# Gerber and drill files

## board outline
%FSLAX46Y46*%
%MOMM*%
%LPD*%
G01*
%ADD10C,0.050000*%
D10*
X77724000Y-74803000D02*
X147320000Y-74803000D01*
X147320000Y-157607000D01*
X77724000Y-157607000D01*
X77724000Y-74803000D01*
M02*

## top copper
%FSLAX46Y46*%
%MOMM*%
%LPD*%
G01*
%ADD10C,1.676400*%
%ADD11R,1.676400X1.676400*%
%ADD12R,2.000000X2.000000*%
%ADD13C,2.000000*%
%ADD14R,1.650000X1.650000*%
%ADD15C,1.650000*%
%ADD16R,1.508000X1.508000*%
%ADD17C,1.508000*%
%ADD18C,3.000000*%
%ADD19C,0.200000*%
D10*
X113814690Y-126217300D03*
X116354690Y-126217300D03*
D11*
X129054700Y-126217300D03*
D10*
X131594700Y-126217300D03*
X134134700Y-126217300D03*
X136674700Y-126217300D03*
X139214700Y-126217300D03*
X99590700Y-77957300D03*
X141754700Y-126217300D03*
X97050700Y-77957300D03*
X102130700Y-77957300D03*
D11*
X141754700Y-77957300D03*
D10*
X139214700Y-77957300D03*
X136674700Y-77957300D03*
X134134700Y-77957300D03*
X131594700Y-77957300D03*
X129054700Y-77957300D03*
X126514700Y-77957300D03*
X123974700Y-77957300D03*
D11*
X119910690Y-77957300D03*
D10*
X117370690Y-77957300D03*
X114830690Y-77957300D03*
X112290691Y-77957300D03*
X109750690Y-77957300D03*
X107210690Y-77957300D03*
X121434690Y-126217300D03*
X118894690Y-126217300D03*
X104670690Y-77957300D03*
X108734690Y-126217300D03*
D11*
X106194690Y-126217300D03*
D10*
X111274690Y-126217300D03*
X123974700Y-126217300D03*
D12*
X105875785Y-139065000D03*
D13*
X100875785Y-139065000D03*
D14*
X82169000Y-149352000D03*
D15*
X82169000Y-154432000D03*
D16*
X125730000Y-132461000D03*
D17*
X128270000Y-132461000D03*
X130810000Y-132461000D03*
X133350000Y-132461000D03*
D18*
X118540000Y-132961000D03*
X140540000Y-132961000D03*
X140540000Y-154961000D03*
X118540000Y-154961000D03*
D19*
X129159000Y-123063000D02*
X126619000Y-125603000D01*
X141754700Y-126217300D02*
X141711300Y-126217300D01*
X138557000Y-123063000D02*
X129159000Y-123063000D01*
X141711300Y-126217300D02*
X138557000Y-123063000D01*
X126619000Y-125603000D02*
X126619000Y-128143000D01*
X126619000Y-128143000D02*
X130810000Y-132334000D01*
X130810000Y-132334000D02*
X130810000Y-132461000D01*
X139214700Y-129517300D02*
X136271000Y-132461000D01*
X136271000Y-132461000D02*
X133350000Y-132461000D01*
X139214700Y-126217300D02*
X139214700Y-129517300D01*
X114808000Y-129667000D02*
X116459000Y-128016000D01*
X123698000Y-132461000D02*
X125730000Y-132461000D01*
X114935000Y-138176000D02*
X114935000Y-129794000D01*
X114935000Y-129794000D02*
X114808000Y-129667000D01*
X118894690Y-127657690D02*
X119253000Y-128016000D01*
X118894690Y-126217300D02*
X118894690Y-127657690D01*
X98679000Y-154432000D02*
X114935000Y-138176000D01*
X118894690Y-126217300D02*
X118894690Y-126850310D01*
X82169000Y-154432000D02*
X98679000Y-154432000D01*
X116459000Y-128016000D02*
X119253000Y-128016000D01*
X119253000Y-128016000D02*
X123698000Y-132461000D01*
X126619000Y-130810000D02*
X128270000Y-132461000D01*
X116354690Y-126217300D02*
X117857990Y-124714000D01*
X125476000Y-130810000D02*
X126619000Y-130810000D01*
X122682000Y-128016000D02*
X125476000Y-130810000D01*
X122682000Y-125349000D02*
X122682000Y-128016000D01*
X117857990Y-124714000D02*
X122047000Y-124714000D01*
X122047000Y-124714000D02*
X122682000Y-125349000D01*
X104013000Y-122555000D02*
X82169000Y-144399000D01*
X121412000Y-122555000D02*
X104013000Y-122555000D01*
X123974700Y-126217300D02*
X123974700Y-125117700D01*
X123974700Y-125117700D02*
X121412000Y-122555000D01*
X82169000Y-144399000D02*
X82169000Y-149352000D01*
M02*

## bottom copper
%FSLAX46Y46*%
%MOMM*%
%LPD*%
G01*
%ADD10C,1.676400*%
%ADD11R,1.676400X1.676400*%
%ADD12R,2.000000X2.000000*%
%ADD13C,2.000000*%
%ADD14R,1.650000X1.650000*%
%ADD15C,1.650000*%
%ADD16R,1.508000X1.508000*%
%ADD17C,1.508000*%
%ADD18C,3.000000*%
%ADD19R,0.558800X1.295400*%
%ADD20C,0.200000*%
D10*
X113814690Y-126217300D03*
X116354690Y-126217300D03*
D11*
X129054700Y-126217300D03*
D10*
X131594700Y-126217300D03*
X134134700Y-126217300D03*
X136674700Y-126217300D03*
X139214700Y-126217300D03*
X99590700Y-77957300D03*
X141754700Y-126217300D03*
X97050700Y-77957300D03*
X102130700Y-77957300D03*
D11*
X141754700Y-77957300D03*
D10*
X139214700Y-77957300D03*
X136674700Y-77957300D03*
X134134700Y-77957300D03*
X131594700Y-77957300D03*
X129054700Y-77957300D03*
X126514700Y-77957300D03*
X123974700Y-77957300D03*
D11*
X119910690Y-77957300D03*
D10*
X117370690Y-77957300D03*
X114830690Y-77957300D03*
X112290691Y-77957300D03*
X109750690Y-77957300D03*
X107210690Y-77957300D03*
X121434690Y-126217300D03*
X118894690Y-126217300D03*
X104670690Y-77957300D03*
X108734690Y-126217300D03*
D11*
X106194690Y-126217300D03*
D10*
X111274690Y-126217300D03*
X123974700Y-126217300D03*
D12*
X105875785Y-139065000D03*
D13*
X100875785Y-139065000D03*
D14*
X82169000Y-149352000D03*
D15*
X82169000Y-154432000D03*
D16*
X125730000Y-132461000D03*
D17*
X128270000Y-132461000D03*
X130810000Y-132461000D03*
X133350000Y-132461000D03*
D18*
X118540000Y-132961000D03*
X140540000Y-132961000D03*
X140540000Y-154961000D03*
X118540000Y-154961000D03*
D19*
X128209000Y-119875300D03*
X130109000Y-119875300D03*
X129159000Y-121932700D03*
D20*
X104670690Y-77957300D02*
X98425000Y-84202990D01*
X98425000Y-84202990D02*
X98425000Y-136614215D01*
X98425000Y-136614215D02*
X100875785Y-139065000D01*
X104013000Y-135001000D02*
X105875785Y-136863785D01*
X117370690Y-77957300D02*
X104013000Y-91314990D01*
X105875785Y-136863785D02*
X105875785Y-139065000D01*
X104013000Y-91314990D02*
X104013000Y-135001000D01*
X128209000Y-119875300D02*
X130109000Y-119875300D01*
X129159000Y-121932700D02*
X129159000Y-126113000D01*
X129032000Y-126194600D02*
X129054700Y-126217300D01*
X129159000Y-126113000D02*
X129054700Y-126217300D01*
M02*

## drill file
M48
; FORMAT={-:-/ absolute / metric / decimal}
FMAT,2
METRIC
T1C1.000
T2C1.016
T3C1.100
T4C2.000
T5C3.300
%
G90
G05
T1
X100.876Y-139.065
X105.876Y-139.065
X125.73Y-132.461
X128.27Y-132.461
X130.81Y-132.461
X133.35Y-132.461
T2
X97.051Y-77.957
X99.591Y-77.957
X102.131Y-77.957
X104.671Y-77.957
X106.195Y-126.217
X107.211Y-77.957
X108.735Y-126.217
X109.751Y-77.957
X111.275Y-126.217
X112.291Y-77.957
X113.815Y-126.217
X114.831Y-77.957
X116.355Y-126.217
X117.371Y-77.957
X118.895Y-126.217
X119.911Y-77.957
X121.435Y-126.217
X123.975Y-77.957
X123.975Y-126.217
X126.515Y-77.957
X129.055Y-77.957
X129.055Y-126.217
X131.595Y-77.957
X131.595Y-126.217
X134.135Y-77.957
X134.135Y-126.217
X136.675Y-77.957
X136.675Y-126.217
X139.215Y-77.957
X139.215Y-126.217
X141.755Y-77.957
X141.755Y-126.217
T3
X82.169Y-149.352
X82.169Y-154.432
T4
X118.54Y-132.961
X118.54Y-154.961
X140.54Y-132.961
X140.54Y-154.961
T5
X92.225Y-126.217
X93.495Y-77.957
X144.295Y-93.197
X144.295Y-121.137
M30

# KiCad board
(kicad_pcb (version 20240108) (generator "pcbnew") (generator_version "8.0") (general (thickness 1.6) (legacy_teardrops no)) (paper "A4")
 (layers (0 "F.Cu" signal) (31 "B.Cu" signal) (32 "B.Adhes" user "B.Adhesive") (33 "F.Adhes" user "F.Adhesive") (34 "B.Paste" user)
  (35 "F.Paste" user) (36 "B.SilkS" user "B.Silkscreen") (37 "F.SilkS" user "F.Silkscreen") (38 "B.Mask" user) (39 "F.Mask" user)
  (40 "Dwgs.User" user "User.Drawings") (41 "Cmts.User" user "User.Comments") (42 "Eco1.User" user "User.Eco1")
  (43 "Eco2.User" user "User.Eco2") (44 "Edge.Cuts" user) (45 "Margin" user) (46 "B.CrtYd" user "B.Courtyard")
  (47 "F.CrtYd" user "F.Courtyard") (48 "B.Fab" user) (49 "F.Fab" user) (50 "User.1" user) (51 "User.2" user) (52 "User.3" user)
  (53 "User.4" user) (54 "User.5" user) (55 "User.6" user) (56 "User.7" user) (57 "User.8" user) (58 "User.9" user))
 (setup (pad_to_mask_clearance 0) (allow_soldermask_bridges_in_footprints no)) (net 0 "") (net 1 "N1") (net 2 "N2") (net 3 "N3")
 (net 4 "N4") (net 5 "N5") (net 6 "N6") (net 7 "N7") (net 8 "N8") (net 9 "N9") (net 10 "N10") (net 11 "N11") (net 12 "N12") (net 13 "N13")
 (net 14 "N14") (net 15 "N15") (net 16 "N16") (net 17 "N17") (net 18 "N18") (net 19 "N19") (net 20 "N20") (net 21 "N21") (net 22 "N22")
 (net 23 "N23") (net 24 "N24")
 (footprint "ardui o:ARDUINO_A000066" (layer "F.Cu") (at 112.522 102.108)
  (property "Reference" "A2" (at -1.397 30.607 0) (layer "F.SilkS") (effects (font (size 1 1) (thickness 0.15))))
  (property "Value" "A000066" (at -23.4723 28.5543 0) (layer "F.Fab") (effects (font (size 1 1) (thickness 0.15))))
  (pad "" np_thru_hole circle (at -20.2973 24.1093) (size 3.3 3.3) (drill 3.3) (layers "*.Cu" "*.Mask"))
  (pad "" np_thru_hole circle (at -19.0273 -24.1507) (size 3.3 3.3) (drill 3.3) (layers "*.Cu" "*.Mask"))
  (pad "" np_thru_hole circle (at 31.7727 -8.91069) (size 3.3 3.3) (drill 3.3) (layers "*.Cu" "*.Mask"))
  (pad "" np_thru_hole circle (at 31.7727 19.0293) (size 3.3 3.3) (drill 3.3) (layers "*.Cu" "*.Mask"))
  (pad "3V3" thru_hole circle (at 1.29269 24.1093) (size 1.6764 1.6764) (drill 1.016) (layers "*.Cu" "*.Mask") (remove_unused_layers no)
   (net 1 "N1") (solder_mask_margin 0.102))
  (pad "5V" thru_hole circle (at 3.83269 24.1093) (size 1.6764 1.6764) (drill 1.016) (layers "*.Cu" "*.Mask") (remove_unused_layers no)
   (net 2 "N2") (solder_mask_margin 0.102))
  (pad "A0" thru_hole rect (at 16.5327 24.1093) (size 1.6764 1.6764) (drill 1.016) (layers "*.Cu" "*.Mask") (remove_unused_layers no)
   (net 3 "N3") (solder_mask_margin 0.102))
  (pad "A1" thru_hole circle (at 19.0727 24.1093) (size 1.6764 1.6764) (drill 1.016) (layers "*.Cu" "*.Mask") (remove_unused_layers no)
   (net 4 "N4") (solder_mask_margin 0.102))
  (pad "A2" thru_hole circle (at 21.6127 24.1093) (size 1.6764 1.6764) (drill 1.016) (layers "*.Cu" "*.Mask") (remove_unused_layers no)
   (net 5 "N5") (solder_mask_margin 0.102))
  (pad "A3" thru_hole circle (at 24.1527 24.1093) (size 1.6764 1.6764) (drill 1.016) (layers "*.Cu" "*.Mask") (remove_unused_layers no)
   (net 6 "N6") (solder_mask_margin 0.102))
  (pad "A4" thru_hole circle (at 26.6927 24.1093) (size 1.6764 1.6764) (drill 1.016) (layers "*.Cu" "*.Mask") (remove_unused_layers no)
   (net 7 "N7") (solder_mask_margin 0.102))
  (pad "A4_SDA" thru_hole circle (at -12.9313 -24.1507) (size 1.6764 1.6764) (drill 1.016) (layers "*.Cu" "*.Mask")
   (remove_unused_layers no) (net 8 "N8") (solder_mask_margin 0.102))
  (pad "A5" thru_hole circle (at 29.2327 24.1093) (size 1.6764 1.6764) (drill 1.016) (layers "*.Cu" "*.Mask") (remove_unused_layers no)
   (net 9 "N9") (solder_mask_margin 0.102))
  (pad "A5_SCL" thru_hole circle (at -15.4713 -24.1507) (size 1.6764 1.6764) (drill 1.016) (layers "*.Cu" "*.Mask")
   (remove_unused_layers no) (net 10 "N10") (solder_mask_margin 0.102))
  (pad "AREF" thru_hole circle (at -10.3913 -24.1507) (size 1.6764 1.6764) (drill 1.016) (layers "*.Cu" "*.Mask") (remove_unused_layers no)
   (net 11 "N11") (solder_mask_margin 0.102))
  (pad "D0" thru_hole rect (at 29.2327 -24.1507) (size 1.6764 1.6764) (drill 1.016) (layers "*.Cu" "*.Mask") (remove_unused_layers no)
   (solder_mask_margin 0.102))
  (pad "D1" thru_hole circle (at 26.6927 -24.1507) (size 1.6764 1.6764) (drill 1.016) (layers "*.Cu" "*.Mask") (remove_unused_layers no)
   (solder_mask_margin 0.102))
  (pad "D2" thru_hole circle (at 24.1527 -24.1507) (size 1.6764 1.6764) (drill 1.016) (layers "*.Cu" "*.Mask") (remove_unused_layers no)
   (solder_mask_margin 0.102))
  (pad "D3" thru_hole circle (at 21.6127 -24.1507) (size 1.6764 1.6764) (drill 1.016) (layers "*.Cu" "*.Mask") (remove_unused_layers no)
   (solder_mask_margin 0.102))
  (pad "D4" thru_hole circle (at 19.0727 -24.1507) (size 1.6764 1.6764) (drill 1.016) (layers "*.Cu" "*.Mask") (remove_unused_layers no)
   (solder_mask_margin 0.102))
  (pad "D5" thru_hole circle (at 16.5327 -24.1507) (size 1.6764 1.6764) (drill 1.016) (layers "*.Cu" "*.Mask") (remove_unused_layers no)
   (solder_mask_margin 0.102))
  (pad "D6" thru_hole circle (at 13.9927 -24.1507) (size 1.6764 1.6764) (drill 1.016) (layers "*.Cu" "*.Mask") (remove_unused_layers no)
   (solder_mask_margin 0.102))
  (pad "D7" thru_hole circle (at 11.4527 -24.1507) (size 1.6764 1.6764) (drill 1.016) (layers "*.Cu" "*.Mask") (remove_unused_layers no)
   (solder_mask_margin 0.102))
  (pad "D8" thru_hole rect (at 7.38869 -24.1507) (size 1.6764 1.6764) (drill 1.016) (layers "*.Cu" "*.Mask") (remove_unused_layers no)
   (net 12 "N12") (solder_mask_margin 0.102))
  (pad "D9" thru_hole circle (at 4.84869 -24.1507) (size 1.6764 1.6764) (drill 1.016) (layers "*.Cu" "*.Mask") (remove_unused_layers no)
   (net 12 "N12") (solder_mask_margin 0.102))
  (pad "D10" thru_hole circle (at 2.30869 -24.1507) (size 1.6764 1.6764) (drill 1.016) (layers "*.Cu" "*.Mask") (remove_unused_layers no)
   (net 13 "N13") (solder_mask_margin 0.102))
  (pad "D11" thru_hole circle (at -0.231309 -24.1507) (size 1.6764 1.6764) (drill 1.016) (layers "*.Cu" "*.Mask") (remove_unused_layers no)
   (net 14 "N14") (solder_mask_margin 0.102))
  (pad "D12" thru_hole circle (at -2.77131 -24.1507) (size 1.6764 1.6764) (drill 1.016) (layers "*.Cu" "*.Mask") (remove_unused_layers no)
   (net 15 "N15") (solder_mask_margin 0.102))
  (pad "D13" thru_hole circle (at -5.31131 -24.1507) (size 1.6764 1.6764) (drill 1.016) (layers "*.Cu" "*.Mask") (remove_unused_layers no)
   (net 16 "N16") (solder_mask_margin 0.102))
  (pad "GND_1" thru_hole circle (at 8.91269 24.1093) (size 1.6764 1.6764) (drill 1.016) (layers "*.Cu" "*.Mask") (remove_unused_layers no)
   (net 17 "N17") (solder_mask_margin 0.102))
  (pad "GND_2" thru_hole circle (at 6.37269 24.1093) (size 1.6764 1.6764) (drill 1.016) (layers "*.Cu" "*.Mask") (remove_unused_layers no)
   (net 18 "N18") (solder_mask_margin 0.102))
  (pad "GND_3" thru_hole circle (at -7.85131 -24.1507) (size 1.6764 1.6764) (drill 1.016) (layers "*.Cu" "*.Mask") (remove_unused_layers no)
   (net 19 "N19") (solder_mask_margin 0.102))
  (pad "IOREF" thru_hole circle (at -3.78731 24.1093) (size 1.6764 1.6764) (drill 1.016) (layers "*.Cu" "*.Mask") (remove_unused_layers no)
   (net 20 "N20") (solder_mask_margin 0.102))
  (pad "P1" thru_hole rect (at -6.32731 24.1093) (size 1.6764 1.6764) (drill 1.016) (layers "*.Cu" "*.Mask") (remove_unused_layers no)
   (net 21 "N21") (solder_mask_margin 0.102))
  (pad "RST" thru_hole circle (at -1.24731 24.1093) (size 1.6764 1.6764) (drill 1.016) (layers "*.Cu" "*.Mask") (remove_unused_layers no)
   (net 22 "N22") (solder_mask_margin 0.102))
  (pad "VIN" thru_hole circle (at 11.4527 24.1093) (size 1.6764 1.6764) (drill 1.016) (layers "*.Cu" "*.Mask") (remove_unused_layers no)
   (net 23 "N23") (solder_mask_margin 0.102)))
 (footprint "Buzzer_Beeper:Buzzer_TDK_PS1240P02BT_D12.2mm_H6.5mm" (layer "F.Cu") (at 105.875785 139.065 180)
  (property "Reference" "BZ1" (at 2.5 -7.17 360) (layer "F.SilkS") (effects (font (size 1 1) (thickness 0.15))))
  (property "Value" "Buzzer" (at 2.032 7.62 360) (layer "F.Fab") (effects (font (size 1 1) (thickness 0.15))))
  (pad "1" thru_hole rect (at 0 0 180) (size 2 2) (drill 1) (layers "*.Cu" "*.Mask") (remove_unused_layers no) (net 12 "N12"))
  (pad "2" thru_hole circle (at 5 0 180) (size 2 2) (drill 1) (layers "*.Cu" "*.Mask") (remove_unused_layers no) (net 19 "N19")))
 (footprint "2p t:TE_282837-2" (layer "F.Cu") (at 82.169 151.892 -90)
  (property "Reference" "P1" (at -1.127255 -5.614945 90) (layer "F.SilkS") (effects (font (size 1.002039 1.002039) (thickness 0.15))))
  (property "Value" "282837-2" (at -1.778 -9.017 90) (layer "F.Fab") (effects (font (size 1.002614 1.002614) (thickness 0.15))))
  (pad "1" thru_hole rect (at -2.54 0 270) (size 1.65 1.65) (drill 1.1) (layers "*.Cu" "*.Mask") (remove_unused_layers no) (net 23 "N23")
   (solder_mask_margin 0.102))
  (pad "2" thru_hole circle (at 2.54 0 270) (size 1.65 1.65) (drill 1.1) (layers "*.Cu" "*.Mask") (remove_unused_layers no) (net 18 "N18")
   (solder_mask_margin 0.102)))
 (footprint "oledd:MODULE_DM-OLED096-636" (layer "F.Cu") (at 129.54 143.961)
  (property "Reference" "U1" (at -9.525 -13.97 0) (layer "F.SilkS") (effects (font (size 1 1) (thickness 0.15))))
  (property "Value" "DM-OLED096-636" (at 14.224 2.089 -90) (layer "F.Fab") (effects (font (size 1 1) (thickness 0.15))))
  (pad "1" thru_hole rect (at -3.81 -11.5) (size 1.508 1.508) (drill 1) (layers "*.Cu" "*.Mask") (remove_unused_layers no) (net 18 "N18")
   (solder_mask_margin 0.102))
  (pad "2" thru_hole circle (at -1.27 -11.5) (size 1.508 1.508) (drill 1) (layers "*.Cu" "*.Mask") (remove_unused_layers no) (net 2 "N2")
   (solder_mask_margin 0.102))
  (pad "3" thru_hole circle (at 1.27 -11.5) (size 1.508 1.508) (drill 1) (layers "*.Cu" "*.Mask") (remove_unused_layers no) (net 9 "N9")
   (solder_mask_margin 0.102))
  (pad "4" thru_hole circle (at 3.81 -11.5) (size 1.508 1.508) (drill 1) (layers "*.Cu" "*.Mask") (remove_unused_layers no) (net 7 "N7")
   (solder_mask_margin 0.102))
  (pad "S1" thru_hole circle (at -11 -11) (size 3 3) (drill 2) (layers "*.Cu" "*.Mask") (remove_unused_layers no) (solder_mask_margin 0.102))
  (pad "S2" thru_hole circle (at 11 -11) (size 3 3) (drill 2) (layers "*.Cu" "*.Mask") (remove_unused_layers no) (solder_mask_margin 0.102))
  (pad "S3" thru_hole circle (at 11 11) (size 3 3) (drill 2) (layers "*.Cu" "*.Mask") (remove_unused_layers no) (solder_mask_margin 0.102))
  (pad "S4" thru_hole circle (at -11 11) (size 3 3) (drill 2) (layers "*.Cu" "*.Mask") (remove_unused_layers no) (solder_mask_margin 0.102)))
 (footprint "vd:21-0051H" (layer "B.Cu") (at 129.159 120.904)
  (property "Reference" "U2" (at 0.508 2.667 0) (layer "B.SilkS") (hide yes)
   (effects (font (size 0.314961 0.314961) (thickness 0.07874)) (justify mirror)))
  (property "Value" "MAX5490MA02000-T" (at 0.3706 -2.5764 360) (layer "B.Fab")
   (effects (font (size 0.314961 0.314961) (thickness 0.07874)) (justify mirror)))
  (pad "1" smd rect (at -0.95 -1.0287) (size 0.5588 1.2954) (layers "B.Cu" "B.Paste" "B.Mask") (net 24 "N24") (solder_mask_margin 0.102))
  (pad "2" smd rect (at 0.95 -1.0287) (size 0.5588 1.2954) (layers "B.Cu" "B.Paste" "B.Mask") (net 24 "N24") (solder_mask_margin 0.102))
  (pad "3" smd rect (at 0 1.0287) (size 0.5588 1.2954) (layers "B.Cu" "B.Paste" "B.Mask") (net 3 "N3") (solder_mask_margin 0.102)))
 (gr_rect (start 77.724 74.803) (end 147.32 157.607) (stroke (width 0.05) (type default)) (fill none) (layer "Edge.Cuts"))
 (segment (start 129.159 123.063) (end 126.619 125.603) (width 0.2) (layer "F.Cu") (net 9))
 (segment (start 141.7547 126.2173) (end 141.7113 126.2173) (width 0.2) (layer "F.Cu") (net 9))
 (segment (start 138.557 123.063) (end 129.159 123.063) (width 0.2) (layer "F.Cu") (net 9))
 (segment (start 141.7113 126.2173) (end 138.557 123.063) (width 0.2) (layer "F.Cu") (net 9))
 (segment (start 126.619 125.603) (end 126.619 128.143) (width 0.2) (layer "F.Cu") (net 9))
 (segment (start 126.619 128.143) (end 130.81 132.334) (width 0.2) (layer "F.Cu") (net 9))
 (segment (start 130.81 132.334) (end 130.81 132.461) (width 0.2) (layer "F.Cu") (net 9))
 (segment (start 139.2147 129.5173) (end 136.271 132.461) (width 0.2) (layer "F.Cu") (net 7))
 (segment (start 136.271 132.461) (end 133.35 132.461) (width 0.2) (layer "F.Cu") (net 7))
 (segment (start 139.2147 126.2173) (end 139.2147 129.5173) (width 0.2) (layer "F.Cu") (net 7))
 (segment (start 104.67069 77.9573) (end 98.425 84.20299) (width 0.2) (layer "B.Cu") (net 19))
 (segment (start 98.425 84.20299) (end 98.425 136.614215) (width 0.2) (layer "B.Cu") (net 19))
 (segment (start 98.425 136.614215) (end 100.875785 139.065) (width 0.2) (layer "B.Cu") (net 19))
 (segment (start 114.808 129.667) (end 116.459 128.016) (width 0.2) (layer "F.Cu") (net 18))
 (segment (start 123.698 132.461) (end 125.73 132.461) (width 0.2) (layer "F.Cu") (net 18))
 (segment (start 114.935 138.176) (end 114.935 129.794) (width 0.2) (layer "F.Cu") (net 18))
 (segment (start 114.935 129.794) (end 114.808 129.667) (width 0.2) (layer "F.Cu") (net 18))
 (segment (start 118.89469 127.65769) (end 119.253 128.016) (width 0.2) (layer "F.Cu") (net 18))
 (segment (start 118.89469 126.2173) (end 118.89469 127.65769) (width 0.2) (layer "F.Cu") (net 18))
 (segment (start 98.679 154.432) (end 114.935 138.176) (width 0.2) (layer "F.Cu") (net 18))
 (segment (start 118.89469 126.2173) (end 118.89469 126.85031) (width 0.2) (layer "F.Cu") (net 18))
 (segment (start 82.169 154.432) (end 98.679 154.432) (width 0.2) (layer "F.Cu") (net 18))
 (segment (start 116.459 128.016) (end 119.253 128.016) (width 0.2) (layer "F.Cu") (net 18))
 (segment (start 119.253 128.016) (end 123.698 132.461) (width 0.2) (layer "F.Cu") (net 18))
 (segment (start 104.013 135.001) (end 105.875785 136.863785) (width 0.2) (layer "B.Cu") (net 12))
 (segment (start 117.37069 77.9573) (end 104.013 91.31499) (width 0.2) (layer "B.Cu") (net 12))
 (segment (start 105.875785 136.863785) (end 105.875785 139.065) (width 0.2) (layer "B.Cu") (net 12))
 (segment (start 104.013 91.31499) (end 104.013 135.001) (width 0.2) (layer "B.Cu") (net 12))
 (segment (start 126.619 130.81) (end 128.27 132.461) (width 0.2) (layer "F.Cu") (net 2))
 (segment (start 116.35469 126.2173) (end 117.85799 124.714) (width 0.2) (layer "F.Cu") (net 2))
 (segment (start 125.476 130.81) (end 126.619 130.81) (width 0.2) (layer "F.Cu") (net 2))
 (segment (start 122.682 128.016) (end 125.476 130.81) (width 0.2) (layer "F.Cu") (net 2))
 (segment (start 122.682 125.349) (end 122.682 128.016) (width 0.2) (layer "F.Cu") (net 2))
 (segment (start 117.85799 124.714) (end 122.047 124.714) (width 0.2) (layer "F.Cu") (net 2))
 (segment (start 122.047 124.714) (end 122.682 125.349) (width 0.2) (layer "F.Cu") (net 2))
 (segment (start 128.209 119.8753) (end 130.109 119.8753) (width 0.2) (layer "B.Cu") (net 24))
 (segment (start 104.013 122.555) (end 82.169 144.399) (width 0.2) (layer "F.Cu") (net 23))
 (segment (start 121.412 122.555) (end 104.013 122.555) (width 0.2) (layer "F.Cu") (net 23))
 (segment (start 123.9747 126.2173) (end 123.9747 125.1177) (width 0.2) (layer "F.Cu") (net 23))
 (segment (start 123.9747 125.1177) (end 121.412 122.555) (width 0.2) (layer "F.Cu") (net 23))
 (segment (start 82.169 144.399) (end 82.169 149.352) (width 0.2) (layer "F.Cu") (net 23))
 (segment (start 129.159 121.9327) (end 129.159 126.113) (width 0.2) (layer "B.Cu") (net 3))
 (segment (start 129.032 126.1946) (end 129.0547 126.2173) (width 0.2) (layer "B.Cu") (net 3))
 (segment (start 129.159 126.113) (end 129.0547 126.2173) (width 0.2) (layer "B.Cu") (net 3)))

